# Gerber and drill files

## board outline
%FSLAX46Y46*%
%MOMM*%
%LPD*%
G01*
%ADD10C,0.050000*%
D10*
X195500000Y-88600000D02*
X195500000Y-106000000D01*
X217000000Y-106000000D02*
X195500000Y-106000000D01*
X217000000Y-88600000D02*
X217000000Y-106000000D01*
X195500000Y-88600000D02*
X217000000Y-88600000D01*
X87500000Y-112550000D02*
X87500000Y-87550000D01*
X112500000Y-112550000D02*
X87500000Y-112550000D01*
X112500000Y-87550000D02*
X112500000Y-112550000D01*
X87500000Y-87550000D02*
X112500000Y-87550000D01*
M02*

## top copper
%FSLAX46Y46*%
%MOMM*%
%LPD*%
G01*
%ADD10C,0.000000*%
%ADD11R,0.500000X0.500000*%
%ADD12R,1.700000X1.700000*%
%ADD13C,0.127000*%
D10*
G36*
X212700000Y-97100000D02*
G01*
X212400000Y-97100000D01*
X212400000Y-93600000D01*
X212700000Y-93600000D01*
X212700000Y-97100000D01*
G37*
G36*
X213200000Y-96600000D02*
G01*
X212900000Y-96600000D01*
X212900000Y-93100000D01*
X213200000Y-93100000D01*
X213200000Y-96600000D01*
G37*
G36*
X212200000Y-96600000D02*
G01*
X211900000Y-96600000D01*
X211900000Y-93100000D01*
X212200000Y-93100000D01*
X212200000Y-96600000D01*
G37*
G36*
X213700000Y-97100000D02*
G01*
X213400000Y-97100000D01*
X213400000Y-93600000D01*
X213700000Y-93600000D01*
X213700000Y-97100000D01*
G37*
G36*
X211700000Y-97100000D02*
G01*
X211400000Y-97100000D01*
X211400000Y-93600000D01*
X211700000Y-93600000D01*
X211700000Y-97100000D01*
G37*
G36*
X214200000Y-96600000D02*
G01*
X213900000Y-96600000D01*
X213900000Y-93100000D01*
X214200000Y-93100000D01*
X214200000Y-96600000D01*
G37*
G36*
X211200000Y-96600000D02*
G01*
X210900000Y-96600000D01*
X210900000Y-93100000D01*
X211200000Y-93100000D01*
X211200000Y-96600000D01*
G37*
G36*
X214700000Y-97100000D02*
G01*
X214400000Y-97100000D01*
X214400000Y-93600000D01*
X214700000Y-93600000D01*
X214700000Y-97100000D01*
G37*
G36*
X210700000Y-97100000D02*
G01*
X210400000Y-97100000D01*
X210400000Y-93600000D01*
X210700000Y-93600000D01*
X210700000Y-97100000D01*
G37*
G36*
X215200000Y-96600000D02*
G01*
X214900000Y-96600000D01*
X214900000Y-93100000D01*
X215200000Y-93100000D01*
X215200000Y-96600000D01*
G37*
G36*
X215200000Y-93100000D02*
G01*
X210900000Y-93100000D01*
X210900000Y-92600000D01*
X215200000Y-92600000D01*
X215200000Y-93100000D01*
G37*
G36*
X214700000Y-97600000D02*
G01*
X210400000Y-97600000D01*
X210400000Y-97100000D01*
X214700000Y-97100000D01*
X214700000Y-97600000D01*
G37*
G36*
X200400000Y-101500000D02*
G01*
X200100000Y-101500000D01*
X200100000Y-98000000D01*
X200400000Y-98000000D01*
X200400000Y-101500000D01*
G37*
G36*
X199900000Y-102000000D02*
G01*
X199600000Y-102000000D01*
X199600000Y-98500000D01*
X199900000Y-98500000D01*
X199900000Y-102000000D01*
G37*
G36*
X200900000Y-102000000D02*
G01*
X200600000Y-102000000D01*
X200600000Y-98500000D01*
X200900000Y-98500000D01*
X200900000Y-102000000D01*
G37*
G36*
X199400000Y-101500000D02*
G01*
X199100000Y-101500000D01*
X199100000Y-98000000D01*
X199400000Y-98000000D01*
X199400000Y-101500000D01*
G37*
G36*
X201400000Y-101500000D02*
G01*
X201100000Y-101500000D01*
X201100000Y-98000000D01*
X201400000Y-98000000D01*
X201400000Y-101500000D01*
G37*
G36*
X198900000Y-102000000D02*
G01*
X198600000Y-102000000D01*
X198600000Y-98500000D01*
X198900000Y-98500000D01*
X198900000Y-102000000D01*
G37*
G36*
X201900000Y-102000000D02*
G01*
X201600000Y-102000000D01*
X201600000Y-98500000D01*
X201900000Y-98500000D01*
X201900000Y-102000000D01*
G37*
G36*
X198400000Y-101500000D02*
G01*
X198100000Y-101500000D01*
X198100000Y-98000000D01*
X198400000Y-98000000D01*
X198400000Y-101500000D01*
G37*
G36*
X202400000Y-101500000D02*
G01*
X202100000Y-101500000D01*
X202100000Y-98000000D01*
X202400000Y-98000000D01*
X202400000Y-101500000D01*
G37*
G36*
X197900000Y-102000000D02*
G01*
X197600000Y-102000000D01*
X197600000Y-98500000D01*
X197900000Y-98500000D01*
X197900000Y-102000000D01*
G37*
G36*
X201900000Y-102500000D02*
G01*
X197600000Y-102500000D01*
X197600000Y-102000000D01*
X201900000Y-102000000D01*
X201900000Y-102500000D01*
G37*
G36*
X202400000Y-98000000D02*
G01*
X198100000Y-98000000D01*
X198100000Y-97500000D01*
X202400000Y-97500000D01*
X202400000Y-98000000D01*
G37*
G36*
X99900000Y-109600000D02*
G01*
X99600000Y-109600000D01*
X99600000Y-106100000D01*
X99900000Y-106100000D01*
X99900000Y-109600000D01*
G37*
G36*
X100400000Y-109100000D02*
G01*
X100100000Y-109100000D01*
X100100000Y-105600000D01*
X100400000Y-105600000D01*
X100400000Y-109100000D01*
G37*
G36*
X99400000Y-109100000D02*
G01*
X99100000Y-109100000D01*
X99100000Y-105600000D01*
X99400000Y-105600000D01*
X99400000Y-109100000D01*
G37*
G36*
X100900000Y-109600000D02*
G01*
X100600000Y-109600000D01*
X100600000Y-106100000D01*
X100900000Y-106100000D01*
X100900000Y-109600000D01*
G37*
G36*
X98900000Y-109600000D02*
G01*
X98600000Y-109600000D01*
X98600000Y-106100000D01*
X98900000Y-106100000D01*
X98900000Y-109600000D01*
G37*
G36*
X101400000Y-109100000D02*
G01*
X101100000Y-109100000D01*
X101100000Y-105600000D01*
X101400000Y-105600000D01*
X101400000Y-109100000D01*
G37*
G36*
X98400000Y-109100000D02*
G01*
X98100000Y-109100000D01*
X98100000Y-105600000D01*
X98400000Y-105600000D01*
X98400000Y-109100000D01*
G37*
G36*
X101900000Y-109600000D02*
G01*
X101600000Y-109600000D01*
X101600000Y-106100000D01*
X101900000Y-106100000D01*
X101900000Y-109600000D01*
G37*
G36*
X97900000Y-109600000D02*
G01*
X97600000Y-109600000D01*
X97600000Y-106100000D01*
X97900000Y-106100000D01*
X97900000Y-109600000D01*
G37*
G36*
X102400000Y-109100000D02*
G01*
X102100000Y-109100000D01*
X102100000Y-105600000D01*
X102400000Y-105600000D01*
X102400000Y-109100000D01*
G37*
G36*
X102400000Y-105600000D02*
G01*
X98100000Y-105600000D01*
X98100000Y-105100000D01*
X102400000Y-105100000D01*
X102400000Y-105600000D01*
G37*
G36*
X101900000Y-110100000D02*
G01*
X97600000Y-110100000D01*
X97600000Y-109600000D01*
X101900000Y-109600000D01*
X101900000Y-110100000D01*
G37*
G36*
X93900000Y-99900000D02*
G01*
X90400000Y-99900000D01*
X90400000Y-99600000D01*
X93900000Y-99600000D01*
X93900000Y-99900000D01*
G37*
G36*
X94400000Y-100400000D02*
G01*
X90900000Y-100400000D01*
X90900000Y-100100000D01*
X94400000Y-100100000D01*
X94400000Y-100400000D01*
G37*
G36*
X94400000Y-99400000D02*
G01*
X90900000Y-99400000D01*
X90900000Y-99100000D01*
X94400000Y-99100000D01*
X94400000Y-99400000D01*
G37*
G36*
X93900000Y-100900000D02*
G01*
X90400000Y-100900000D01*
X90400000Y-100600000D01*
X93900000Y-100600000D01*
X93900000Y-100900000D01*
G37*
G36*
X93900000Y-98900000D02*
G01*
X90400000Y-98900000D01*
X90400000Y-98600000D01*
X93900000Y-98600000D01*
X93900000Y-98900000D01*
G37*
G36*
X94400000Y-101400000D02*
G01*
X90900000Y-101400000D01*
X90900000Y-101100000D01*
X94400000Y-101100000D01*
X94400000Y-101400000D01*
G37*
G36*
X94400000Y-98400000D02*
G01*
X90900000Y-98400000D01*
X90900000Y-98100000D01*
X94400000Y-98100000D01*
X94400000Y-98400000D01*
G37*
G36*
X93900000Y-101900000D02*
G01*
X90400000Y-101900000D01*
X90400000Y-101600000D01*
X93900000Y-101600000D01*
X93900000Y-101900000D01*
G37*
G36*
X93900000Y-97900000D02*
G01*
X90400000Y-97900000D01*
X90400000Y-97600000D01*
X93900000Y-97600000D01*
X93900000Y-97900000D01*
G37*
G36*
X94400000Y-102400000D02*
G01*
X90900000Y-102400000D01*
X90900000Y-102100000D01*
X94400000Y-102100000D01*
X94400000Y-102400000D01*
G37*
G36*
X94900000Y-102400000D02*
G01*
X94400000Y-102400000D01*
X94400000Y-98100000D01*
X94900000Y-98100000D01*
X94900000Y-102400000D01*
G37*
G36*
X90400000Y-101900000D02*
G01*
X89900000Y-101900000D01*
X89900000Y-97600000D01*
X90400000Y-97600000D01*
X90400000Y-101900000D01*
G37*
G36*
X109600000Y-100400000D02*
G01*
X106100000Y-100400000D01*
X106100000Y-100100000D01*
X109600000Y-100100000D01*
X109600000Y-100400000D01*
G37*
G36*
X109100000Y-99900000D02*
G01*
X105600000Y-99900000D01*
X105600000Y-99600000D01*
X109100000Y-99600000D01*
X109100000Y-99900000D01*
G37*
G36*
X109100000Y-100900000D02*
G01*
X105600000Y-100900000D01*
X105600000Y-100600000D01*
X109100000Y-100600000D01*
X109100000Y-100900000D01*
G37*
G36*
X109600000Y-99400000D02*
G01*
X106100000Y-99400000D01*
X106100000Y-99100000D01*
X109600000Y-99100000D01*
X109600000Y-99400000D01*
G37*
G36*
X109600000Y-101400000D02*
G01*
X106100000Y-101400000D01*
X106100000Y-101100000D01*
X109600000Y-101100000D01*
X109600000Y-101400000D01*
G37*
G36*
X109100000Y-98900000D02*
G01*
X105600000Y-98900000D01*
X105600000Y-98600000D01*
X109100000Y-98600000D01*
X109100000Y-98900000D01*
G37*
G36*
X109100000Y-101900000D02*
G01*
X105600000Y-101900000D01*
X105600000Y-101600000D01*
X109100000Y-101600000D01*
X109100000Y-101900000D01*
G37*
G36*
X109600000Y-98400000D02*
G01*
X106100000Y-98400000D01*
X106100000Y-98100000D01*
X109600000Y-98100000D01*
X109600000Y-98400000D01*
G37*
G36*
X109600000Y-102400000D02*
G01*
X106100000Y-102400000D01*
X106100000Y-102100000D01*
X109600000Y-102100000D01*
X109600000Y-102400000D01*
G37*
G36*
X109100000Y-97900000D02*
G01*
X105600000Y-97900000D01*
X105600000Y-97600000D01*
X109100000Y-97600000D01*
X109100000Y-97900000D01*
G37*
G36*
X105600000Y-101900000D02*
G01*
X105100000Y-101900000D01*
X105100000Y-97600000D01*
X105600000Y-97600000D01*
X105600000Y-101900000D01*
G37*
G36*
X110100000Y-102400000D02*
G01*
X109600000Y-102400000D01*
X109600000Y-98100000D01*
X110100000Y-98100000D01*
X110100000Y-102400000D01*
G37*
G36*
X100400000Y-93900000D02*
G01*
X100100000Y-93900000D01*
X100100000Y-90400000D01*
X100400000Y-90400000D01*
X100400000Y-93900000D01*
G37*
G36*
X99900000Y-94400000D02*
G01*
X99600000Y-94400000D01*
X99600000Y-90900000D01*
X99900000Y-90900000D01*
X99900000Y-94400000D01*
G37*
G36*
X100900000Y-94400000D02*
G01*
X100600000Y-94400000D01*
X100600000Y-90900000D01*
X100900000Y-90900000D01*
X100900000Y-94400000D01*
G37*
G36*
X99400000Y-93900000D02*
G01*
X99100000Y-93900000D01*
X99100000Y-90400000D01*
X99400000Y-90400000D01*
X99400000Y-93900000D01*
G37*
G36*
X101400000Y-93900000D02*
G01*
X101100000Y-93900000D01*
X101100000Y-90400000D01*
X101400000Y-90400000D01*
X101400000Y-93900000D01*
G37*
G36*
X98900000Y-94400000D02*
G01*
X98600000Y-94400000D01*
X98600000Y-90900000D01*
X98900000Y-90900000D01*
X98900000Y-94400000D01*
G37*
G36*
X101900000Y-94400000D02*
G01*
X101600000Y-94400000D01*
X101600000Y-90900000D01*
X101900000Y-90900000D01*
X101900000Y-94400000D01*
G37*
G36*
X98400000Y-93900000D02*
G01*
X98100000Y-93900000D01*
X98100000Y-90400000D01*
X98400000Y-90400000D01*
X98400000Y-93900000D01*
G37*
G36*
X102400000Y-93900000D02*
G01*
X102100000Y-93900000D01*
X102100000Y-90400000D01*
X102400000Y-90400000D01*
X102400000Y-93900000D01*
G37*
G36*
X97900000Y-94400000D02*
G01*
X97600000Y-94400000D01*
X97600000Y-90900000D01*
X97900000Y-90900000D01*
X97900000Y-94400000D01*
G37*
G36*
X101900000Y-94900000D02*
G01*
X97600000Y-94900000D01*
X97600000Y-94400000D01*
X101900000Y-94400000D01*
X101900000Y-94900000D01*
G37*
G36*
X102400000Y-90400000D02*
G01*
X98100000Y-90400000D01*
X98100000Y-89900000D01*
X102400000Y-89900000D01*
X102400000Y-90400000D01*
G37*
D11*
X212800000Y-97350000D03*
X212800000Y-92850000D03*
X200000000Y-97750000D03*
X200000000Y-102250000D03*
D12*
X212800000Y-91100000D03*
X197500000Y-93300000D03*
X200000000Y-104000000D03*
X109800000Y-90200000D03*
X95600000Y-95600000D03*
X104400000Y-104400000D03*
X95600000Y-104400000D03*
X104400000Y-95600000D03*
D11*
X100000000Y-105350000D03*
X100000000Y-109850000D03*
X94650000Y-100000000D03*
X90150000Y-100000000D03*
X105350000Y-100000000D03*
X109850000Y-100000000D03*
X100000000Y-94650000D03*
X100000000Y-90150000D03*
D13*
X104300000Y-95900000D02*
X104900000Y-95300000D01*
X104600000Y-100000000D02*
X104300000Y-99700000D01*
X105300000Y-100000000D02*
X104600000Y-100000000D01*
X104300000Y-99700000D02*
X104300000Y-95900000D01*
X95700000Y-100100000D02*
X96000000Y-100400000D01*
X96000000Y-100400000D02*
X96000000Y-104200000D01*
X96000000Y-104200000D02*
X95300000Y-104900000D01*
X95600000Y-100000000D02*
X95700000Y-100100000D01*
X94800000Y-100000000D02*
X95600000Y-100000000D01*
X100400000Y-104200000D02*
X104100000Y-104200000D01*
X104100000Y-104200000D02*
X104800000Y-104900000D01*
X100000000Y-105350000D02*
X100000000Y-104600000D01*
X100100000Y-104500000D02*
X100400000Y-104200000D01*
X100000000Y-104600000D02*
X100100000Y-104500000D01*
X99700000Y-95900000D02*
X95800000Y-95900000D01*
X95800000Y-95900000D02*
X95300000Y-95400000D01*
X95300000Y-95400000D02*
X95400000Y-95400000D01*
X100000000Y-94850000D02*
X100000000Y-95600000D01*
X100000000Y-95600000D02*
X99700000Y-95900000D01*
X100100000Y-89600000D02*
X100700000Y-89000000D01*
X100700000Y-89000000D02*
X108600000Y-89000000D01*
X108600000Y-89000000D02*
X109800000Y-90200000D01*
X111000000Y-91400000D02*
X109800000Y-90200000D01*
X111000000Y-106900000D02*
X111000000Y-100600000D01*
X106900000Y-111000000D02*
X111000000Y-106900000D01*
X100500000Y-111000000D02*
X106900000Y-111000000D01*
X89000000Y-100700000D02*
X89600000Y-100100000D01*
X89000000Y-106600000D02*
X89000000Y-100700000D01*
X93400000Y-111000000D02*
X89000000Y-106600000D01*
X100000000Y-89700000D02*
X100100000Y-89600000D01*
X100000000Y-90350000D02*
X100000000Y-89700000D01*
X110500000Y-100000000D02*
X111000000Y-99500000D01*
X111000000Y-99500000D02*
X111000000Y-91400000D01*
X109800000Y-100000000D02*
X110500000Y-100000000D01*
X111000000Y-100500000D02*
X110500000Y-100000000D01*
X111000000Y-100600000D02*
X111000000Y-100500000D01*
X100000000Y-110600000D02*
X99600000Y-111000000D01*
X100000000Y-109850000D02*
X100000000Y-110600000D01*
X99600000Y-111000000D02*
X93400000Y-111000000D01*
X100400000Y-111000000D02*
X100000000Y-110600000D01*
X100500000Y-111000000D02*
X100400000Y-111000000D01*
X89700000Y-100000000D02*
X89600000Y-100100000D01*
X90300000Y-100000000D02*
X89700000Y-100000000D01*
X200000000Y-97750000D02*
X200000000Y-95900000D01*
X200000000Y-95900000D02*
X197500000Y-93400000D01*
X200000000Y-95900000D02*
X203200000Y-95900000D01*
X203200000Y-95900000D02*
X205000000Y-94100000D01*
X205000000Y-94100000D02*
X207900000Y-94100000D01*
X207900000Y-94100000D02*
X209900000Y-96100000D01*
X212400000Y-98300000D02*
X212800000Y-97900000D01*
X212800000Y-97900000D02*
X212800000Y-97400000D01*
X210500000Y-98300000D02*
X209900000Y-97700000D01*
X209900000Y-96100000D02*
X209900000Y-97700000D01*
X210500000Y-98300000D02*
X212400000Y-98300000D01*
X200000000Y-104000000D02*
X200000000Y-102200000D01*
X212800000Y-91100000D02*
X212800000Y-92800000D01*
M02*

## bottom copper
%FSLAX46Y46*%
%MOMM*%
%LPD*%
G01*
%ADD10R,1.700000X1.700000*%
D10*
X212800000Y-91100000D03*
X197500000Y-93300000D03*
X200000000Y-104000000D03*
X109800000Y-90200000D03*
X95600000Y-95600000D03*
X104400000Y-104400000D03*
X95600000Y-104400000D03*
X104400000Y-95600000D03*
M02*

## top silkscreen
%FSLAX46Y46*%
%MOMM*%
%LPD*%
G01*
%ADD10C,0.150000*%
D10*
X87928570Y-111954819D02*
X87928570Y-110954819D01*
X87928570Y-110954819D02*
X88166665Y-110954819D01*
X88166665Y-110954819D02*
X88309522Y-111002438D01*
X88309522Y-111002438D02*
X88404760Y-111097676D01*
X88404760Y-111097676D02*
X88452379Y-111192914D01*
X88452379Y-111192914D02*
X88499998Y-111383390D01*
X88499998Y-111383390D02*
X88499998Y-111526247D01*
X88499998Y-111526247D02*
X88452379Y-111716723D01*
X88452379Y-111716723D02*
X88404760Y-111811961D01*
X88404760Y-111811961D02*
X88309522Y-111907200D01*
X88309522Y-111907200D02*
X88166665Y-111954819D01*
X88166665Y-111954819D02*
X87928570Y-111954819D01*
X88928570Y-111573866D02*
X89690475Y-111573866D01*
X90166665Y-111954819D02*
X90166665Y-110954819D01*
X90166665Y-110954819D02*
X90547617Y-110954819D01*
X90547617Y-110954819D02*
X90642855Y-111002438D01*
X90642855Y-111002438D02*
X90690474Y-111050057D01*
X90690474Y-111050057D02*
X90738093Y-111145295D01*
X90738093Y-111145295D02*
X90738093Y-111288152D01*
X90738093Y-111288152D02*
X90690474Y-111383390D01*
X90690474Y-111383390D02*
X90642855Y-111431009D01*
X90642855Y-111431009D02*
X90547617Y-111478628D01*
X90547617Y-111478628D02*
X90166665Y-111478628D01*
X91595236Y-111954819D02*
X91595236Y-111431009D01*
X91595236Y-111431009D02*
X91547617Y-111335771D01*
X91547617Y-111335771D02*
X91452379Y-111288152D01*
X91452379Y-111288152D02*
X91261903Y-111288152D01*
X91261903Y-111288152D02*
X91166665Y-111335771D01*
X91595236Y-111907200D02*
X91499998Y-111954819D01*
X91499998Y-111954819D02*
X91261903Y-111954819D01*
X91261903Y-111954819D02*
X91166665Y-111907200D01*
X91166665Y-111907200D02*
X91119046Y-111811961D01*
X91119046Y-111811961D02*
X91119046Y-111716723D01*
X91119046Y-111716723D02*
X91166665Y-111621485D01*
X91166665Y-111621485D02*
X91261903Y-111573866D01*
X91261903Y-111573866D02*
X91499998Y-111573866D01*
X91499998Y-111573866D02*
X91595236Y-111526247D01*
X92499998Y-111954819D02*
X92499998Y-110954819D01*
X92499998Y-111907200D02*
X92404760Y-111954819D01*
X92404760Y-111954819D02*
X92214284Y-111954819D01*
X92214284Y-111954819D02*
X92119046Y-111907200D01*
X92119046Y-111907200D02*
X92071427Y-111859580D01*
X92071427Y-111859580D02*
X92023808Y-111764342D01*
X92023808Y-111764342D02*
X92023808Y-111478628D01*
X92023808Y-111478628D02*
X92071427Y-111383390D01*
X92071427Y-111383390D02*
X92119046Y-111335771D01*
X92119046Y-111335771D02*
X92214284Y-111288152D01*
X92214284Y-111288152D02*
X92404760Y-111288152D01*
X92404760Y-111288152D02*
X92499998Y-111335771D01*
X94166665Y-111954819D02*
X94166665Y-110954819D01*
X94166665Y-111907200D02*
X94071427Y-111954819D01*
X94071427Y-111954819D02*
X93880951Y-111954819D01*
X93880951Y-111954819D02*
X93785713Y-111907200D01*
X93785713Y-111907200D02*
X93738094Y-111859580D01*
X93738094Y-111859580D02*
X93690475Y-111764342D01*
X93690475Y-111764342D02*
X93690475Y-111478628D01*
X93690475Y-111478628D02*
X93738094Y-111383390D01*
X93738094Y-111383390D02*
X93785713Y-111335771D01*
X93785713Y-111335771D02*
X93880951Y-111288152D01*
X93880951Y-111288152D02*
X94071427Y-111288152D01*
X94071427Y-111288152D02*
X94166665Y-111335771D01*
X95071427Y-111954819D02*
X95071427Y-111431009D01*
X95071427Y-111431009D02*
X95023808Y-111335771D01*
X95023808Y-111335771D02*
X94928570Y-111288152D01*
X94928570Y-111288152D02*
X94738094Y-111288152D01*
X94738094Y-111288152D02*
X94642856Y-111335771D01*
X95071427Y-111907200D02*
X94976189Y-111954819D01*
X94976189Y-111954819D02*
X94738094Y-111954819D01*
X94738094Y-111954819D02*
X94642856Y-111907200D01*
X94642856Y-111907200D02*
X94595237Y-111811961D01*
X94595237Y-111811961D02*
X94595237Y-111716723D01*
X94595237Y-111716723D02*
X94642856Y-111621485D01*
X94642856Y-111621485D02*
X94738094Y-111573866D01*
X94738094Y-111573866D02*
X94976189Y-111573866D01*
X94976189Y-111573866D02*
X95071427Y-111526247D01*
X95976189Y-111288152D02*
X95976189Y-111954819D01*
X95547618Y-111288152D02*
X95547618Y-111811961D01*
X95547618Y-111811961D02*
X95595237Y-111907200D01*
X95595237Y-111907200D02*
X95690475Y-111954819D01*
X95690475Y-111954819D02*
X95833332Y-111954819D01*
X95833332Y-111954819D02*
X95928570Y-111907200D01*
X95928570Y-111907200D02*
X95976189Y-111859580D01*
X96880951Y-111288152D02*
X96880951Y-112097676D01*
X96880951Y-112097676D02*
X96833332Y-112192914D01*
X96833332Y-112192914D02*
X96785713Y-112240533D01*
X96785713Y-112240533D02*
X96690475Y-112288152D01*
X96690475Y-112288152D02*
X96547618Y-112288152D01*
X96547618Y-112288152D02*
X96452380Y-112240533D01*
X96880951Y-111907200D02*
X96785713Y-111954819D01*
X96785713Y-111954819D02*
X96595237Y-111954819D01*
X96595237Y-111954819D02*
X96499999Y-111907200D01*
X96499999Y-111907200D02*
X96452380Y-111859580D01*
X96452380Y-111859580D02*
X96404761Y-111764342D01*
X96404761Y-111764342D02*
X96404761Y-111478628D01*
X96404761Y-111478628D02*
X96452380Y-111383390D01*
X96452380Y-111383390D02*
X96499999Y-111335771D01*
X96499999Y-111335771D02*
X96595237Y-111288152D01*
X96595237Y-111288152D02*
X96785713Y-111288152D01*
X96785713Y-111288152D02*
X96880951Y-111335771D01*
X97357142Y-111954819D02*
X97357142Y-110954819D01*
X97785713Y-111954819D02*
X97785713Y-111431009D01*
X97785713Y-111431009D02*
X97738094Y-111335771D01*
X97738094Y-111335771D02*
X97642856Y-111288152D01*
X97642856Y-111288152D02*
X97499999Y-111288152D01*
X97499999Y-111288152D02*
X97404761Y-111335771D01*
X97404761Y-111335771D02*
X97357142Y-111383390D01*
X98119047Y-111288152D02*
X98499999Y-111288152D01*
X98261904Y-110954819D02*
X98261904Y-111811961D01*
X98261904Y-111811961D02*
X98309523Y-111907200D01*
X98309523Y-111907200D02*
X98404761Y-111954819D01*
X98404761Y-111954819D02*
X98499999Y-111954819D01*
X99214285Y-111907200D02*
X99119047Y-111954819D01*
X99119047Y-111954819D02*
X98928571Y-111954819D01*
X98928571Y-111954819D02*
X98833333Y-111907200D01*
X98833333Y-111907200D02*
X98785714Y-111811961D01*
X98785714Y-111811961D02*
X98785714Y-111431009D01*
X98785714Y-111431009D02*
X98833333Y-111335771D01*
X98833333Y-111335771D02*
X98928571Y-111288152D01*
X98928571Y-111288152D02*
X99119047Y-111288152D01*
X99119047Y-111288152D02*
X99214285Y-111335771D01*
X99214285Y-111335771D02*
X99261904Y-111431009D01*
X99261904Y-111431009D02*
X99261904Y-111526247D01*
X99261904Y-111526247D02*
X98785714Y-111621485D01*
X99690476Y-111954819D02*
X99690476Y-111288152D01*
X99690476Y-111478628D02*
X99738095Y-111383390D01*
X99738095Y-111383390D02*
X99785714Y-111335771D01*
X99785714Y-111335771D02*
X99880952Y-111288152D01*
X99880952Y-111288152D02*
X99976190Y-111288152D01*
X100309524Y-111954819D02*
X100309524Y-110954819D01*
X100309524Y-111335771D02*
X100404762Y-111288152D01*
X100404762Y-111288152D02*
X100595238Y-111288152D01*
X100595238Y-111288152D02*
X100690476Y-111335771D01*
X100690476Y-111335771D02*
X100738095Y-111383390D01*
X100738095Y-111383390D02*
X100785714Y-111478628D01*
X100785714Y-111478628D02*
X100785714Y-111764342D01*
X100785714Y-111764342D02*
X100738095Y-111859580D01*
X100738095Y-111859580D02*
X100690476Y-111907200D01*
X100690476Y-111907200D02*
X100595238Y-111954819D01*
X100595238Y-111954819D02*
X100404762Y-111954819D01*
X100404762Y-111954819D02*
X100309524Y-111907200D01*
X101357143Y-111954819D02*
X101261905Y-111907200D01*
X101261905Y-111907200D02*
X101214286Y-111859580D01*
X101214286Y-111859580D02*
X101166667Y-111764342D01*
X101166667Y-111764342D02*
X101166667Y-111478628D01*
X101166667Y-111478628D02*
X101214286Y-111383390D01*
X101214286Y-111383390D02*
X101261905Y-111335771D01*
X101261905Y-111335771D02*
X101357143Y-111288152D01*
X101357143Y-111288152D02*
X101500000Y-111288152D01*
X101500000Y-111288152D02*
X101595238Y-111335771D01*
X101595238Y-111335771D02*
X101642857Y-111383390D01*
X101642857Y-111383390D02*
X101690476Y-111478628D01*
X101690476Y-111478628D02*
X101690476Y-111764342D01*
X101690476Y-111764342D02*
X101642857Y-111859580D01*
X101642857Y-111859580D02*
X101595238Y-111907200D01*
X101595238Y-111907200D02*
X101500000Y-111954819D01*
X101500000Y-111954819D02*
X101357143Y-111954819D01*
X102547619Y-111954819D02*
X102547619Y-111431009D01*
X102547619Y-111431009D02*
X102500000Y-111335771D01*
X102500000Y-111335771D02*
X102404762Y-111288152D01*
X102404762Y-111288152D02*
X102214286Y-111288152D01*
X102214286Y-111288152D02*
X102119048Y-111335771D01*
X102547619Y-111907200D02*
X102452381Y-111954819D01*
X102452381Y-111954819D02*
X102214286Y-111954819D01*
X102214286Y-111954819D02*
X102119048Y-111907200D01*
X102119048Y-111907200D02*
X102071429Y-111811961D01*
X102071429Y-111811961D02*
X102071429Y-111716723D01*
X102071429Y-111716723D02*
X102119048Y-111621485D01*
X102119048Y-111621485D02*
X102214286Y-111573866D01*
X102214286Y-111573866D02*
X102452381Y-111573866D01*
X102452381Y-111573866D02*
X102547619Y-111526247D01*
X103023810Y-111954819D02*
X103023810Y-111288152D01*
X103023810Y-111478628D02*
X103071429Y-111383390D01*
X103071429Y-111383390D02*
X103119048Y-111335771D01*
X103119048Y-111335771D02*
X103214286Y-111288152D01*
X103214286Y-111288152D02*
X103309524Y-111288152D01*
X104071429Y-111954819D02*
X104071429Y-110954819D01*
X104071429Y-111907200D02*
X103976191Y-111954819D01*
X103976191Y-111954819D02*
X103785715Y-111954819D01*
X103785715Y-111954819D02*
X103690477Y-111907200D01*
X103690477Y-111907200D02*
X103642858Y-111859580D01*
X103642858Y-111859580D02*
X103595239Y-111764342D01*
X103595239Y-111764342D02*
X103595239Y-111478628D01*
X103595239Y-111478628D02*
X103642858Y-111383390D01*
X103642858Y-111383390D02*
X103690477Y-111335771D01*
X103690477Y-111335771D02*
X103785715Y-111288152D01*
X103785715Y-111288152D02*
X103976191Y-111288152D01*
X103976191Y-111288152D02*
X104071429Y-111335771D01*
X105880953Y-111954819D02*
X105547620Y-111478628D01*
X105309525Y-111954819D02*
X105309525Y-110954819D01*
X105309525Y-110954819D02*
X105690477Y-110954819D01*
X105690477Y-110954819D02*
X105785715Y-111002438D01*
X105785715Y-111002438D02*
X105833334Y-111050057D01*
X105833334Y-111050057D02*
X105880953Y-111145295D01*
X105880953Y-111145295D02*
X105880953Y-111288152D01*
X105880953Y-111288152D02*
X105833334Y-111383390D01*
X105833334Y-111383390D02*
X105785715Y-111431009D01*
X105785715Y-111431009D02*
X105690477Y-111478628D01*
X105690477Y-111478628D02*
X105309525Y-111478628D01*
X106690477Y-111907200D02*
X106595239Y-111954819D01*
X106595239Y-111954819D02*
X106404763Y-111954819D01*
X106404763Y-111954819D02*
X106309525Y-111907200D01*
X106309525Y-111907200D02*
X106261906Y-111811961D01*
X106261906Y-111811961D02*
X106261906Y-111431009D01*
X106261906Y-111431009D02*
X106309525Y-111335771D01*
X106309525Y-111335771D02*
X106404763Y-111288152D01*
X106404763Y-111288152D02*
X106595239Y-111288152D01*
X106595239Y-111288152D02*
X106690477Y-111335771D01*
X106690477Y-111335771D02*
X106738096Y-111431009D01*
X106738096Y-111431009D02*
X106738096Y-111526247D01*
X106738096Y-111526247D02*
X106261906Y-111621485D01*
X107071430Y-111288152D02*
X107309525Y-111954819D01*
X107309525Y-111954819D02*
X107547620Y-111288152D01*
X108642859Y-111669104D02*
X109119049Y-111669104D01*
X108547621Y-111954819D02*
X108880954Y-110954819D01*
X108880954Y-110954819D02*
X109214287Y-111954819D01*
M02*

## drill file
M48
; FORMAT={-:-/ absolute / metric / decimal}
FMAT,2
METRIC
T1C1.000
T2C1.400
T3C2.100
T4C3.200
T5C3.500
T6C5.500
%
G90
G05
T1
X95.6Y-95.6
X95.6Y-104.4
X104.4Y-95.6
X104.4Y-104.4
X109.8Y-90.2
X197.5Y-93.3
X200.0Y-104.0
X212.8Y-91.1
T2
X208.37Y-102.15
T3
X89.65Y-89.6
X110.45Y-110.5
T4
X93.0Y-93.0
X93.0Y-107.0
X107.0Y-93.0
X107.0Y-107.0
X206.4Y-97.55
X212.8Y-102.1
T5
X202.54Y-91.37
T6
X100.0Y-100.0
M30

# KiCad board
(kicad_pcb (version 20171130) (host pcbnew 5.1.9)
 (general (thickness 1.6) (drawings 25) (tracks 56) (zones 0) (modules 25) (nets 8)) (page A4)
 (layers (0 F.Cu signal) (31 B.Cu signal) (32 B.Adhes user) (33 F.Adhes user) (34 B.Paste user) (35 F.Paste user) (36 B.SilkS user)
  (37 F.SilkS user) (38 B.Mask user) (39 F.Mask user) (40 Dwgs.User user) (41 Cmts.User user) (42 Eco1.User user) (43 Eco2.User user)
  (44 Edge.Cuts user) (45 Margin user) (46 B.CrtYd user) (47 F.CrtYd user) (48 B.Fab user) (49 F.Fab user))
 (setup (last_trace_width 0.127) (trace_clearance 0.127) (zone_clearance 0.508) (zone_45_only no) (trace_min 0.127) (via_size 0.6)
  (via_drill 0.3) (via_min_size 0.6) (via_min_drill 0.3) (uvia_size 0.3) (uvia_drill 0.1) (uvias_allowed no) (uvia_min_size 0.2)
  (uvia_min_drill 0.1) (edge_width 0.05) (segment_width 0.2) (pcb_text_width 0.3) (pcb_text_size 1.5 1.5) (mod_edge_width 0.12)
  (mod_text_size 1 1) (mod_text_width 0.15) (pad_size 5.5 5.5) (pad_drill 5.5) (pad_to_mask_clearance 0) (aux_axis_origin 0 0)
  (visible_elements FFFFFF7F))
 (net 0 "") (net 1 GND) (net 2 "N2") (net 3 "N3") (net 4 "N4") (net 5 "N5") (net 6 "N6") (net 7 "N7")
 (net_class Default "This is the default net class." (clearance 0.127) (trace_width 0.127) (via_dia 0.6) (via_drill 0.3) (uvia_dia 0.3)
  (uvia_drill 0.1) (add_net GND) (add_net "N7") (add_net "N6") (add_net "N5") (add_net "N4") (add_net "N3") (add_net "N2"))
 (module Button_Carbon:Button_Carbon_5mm (layer F.Cu) (at 212.8 95.1)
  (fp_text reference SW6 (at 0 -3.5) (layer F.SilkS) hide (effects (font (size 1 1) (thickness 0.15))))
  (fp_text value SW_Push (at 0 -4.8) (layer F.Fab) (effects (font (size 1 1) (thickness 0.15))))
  (fp_poly (pts (xy -0.1 2) (xy -0.4 2) (xy -0.4 -1.5) (xy -0.1 -1.5)) (layer F.Cu) (width 0))
  (fp_poly (pts (xy 0.4 1.5) (xy 0.1 1.5) (xy 0.1 -2) (xy 0.4 -2)) (layer F.Cu) (width 0))
  (fp_poly (pts (xy -0.6 1.5) (xy -0.9 1.5) (xy -0.9 -2) (xy -0.6 -2)) (layer F.Cu) (width 0))
  (fp_poly (pts (xy 0.9 2) (xy 0.6 2) (xy 0.6 -1.5) (xy 0.9 -1.5)) (layer F.Cu) (width 0))
  (fp_poly (pts (xy -1.1 2) (xy -1.4 2) (xy -1.4 -1.5) (xy -1.1 -1.5)) (layer F.Cu) (width 0))
  (fp_poly (pts (xy 1.4 1.5) (xy 1.1 1.5) (xy 1.1 -2) (xy 1.4 -2)) (layer F.Cu) (width 0))
  (fp_poly (pts (xy -1.6 1.5) (xy -1.9 1.5) (xy -1.9 -2) (xy -1.6 -2)) (layer F.Cu) (width 0))
  (fp_poly (pts (xy 1.9 2) (xy 1.6 2) (xy 1.6 -1.5) (xy 1.9 -1.5)) (layer F.Cu) (width 0))
  (fp_poly (pts (xy -2.1 2) (xy -2.4 2) (xy -2.4 -1.5) (xy -2.1 -1.5)) (layer F.Cu) (width 0))
  (fp_poly (pts (xy 2.4 1.5) (xy 2.1 1.5) (xy 2.1 -2) (xy 2.4 -2)) (layer F.Cu) (width 0))
  (fp_poly (pts (xy 2.4 -2.5) (xy 2.4 -2) (xy -1.9 -2) (xy -1.9 -2.5)) (layer F.Cu) (width 0))
  (fp_poly (pts (xy 1.9 2) (xy 1.9 2.5) (xy -2.4 2.5) (xy -2.4 2)) (layer F.Cu) (width 0))
  (pad 2 smd rect (at 0 2.25) (size 0.5 0.5) (layers F.Cu F.Mask) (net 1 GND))
  (pad 1 smd rect (at 0 -2.25) (size 0.5 0.5) (layers F.Cu F.Mask) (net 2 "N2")))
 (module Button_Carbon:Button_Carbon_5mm (layer F.Cu) (at 200 100 180)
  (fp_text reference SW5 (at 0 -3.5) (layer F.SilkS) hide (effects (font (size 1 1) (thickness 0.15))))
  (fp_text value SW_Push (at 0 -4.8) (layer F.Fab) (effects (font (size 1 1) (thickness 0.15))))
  (fp_poly (pts (xy -0.1 2) (xy -0.4 2) (xy -0.4 -1.5) (xy -0.1 -1.5)) (layer F.Cu) (width 0))
  (fp_poly (pts (xy 0.4 1.5) (xy 0.1 1.5) (xy 0.1 -2) (xy 0.4 -2)) (layer F.Cu) (width 0))
  (fp_poly (pts (xy -0.6 1.5) (xy -0.9 1.5) (xy -0.9 -2) (xy -0.6 -2)) (layer F.Cu) (width 0))
  (fp_poly (pts (xy 0.9 2) (xy 0.6 2) (xy 0.6 -1.5) (xy 0.9 -1.5)) (layer F.Cu) (width 0))
  (fp_poly (pts (xy -1.1 2) (xy -1.4 2) (xy -1.4 -1.5) (xy -1.1 -1.5)) (layer F.Cu) (width 0))
  (fp_poly (pts (xy 1.4 1.5) (xy 1.1 1.5) (xy 1.1 -2) (xy 1.4 -2)) (layer F.Cu) (width 0))
  (fp_poly (pts (xy -1.6 1.5) (xy -1.9 1.5) (xy -1.9 -2) (xy -1.6 -2)) (layer F.Cu) (width 0))
  (fp_poly (pts (xy 1.9 2) (xy 1.6 2) (xy 1.6 -1.5) (xy 1.9 -1.5)) (layer F.Cu) (width 0))
  (fp_poly (pts (xy -2.1 2) (xy -2.4 2) (xy -2.4 -1.5) (xy -2.1 -1.5)) (layer F.Cu) (width 0))
  (fp_poly (pts (xy 2.4 1.5) (xy 2.1 1.5) (xy 2.1 -2) (xy 2.4 -2)) (layer F.Cu) (width 0))
  (fp_poly (pts (xy 2.4 -2.5) (xy 2.4 -2) (xy -1.9 -2) (xy -1.9 -2.5)) (layer F.Cu) (width 0))
  (fp_poly (pts (xy 1.9 2) (xy 1.9 2.5) (xy -2.4 2.5) (xy -2.4 2)) (layer F.Cu) (width 0))
  (pad 2 smd rect (at 0 2.25 180) (size 0.5 0.5) (layers F.Cu F.Mask) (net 1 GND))
  (pad 1 smd rect (at 0 -2.25 180) (size 0.5 0.5) (layers F.Cu F.Mask) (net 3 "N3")))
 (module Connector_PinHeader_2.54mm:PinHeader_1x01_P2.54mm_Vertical (layer B.Cu) (at 212.8 91.1)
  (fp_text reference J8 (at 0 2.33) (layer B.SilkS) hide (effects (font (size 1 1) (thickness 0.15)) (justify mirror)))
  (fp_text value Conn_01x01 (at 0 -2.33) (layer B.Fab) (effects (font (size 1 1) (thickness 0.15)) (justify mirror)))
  (pad 1 thru_hole rect (at 0 0) (size 1.7 1.7) (drill 1) (layers *.Cu *.Mask) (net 2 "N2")))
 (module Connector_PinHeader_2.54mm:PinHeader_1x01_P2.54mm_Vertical (layer B.Cu) (at 197.5 93.3)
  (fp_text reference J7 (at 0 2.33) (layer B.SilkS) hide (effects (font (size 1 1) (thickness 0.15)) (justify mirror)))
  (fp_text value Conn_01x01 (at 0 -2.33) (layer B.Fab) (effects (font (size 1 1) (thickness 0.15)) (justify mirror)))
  (pad 1 thru_hole rect (at 0 0) (size 1.7 1.7) (drill 1) (layers *.Cu *.Mask) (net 1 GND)))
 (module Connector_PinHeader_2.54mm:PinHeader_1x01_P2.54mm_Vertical (layer B.Cu) (at 200 104)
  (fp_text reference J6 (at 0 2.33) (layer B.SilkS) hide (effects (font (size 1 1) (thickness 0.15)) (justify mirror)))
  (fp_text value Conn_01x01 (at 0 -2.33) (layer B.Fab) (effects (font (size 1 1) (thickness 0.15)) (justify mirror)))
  (pad 1 thru_hole rect (at 0 0) (size 1.7 1.7) (drill 1) (layers *.Cu *.Mask) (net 3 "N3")))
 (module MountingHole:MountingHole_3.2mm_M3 (layer F.Cu) (at 212.8 102.1)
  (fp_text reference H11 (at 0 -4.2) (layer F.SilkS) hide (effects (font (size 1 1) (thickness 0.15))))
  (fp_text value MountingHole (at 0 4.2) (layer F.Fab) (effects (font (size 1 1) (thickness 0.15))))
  (pad 1 np_thru_hole circle (at 0 0) (size 3.2 3.2) (drill 3.2) (layers *.Cu *.Mask)))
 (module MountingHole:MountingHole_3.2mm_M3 (layer F.Cu) (at 206.4 97.55)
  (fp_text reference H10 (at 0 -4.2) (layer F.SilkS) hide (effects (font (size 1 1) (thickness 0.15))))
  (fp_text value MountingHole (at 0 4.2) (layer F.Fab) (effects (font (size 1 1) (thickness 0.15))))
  (pad 1 np_thru_hole circle (at 0 0) (size 3.2 3.2) (drill 3.2) (layers *.Cu *.Mask)))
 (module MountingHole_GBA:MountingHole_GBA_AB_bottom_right (layer F.Cu) (at 208.37 102.15)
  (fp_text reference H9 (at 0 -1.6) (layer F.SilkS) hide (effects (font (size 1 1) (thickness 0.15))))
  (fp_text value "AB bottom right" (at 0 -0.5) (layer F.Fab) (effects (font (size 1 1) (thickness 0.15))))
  (pad "" np_thru_hole circle (at 0 0 180) (size 1.4 1.4) (drill 1.4) (layers *.Cu *.Mask)))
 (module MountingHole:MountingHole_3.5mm (layer F.Cu) (at 202.54 91.37)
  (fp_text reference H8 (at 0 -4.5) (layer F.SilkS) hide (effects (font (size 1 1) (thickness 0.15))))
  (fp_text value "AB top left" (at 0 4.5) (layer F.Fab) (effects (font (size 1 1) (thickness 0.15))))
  (pad 1 np_thru_hole circle (at 0 0) (size 3.5 3.5) (drill 3.5) (layers *.Cu *.Mask)))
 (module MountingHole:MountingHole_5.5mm (layer F.Cu) (at 100 100)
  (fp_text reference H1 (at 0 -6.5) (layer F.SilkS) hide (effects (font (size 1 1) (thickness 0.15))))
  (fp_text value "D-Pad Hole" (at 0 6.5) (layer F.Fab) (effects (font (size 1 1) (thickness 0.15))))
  (pad 1 np_thru_hole circle (at 0 0) (size 5.5 5.5) (drill 5.5) (layers *.Cu *.Mask)))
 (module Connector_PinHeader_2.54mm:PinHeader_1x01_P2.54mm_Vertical (layer B.Cu) (at 109.8 90.2)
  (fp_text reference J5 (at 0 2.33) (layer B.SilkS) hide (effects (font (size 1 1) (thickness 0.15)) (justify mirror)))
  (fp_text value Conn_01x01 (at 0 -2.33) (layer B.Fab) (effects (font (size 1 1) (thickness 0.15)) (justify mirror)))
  (pad 1 thru_hole rect (at 0 0) (size 1.7 1.7) (drill 1) (layers *.Cu *.Mask) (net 1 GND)))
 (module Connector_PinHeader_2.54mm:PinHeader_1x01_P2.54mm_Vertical (layer B.Cu) (at 95.6 95.6)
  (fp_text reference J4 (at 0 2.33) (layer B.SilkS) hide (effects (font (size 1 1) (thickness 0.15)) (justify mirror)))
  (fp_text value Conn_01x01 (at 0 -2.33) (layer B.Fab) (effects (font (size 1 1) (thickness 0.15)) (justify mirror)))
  (pad 1 thru_hole rect (at 0 0) (size 1.7 1.7) (drill 1) (layers *.Cu *.Mask) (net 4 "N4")))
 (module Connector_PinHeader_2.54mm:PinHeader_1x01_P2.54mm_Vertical (layer B.Cu) (at 104.4 104.4)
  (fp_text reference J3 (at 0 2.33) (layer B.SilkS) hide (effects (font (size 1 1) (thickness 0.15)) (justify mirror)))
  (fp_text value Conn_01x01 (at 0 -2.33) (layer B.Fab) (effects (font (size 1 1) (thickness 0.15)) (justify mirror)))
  (pad 1 thru_hole rect (at 0 0) (size 1.7 1.7) (drill 1) (layers *.Cu *.Mask) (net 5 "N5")))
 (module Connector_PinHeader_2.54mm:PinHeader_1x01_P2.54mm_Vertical (layer B.Cu) (at 95.6 104.4)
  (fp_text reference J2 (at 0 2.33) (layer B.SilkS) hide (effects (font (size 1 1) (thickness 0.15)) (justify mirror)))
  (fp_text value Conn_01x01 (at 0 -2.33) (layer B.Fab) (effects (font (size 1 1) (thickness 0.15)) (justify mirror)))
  (pad 1 thru_hole rect (at 0 0) (size 1.7 1.7) (drill 1) (layers *.Cu *.Mask) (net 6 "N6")))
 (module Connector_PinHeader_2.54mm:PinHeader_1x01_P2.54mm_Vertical (layer B.Cu) (at 104.4 95.6)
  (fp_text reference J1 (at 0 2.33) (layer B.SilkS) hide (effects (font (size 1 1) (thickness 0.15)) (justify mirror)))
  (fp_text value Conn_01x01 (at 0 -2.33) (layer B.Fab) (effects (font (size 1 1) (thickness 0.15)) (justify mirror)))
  (pad 1 thru_hole rect (at 0 0) (size 1.7 1.7) (drill 1) (layers *.Cu *.Mask) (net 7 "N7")))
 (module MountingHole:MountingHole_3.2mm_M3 (layer F.Cu) (at 93 107)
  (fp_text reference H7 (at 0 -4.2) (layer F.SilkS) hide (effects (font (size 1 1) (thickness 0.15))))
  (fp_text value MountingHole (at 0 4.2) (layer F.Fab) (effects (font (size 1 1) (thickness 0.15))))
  (pad 1 np_thru_hole circle (at 0 0) (size 3.2 3.2) (drill 3.2) (layers *.Cu *.Mask)))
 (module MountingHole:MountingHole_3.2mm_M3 (layer F.Cu) (at 107 93)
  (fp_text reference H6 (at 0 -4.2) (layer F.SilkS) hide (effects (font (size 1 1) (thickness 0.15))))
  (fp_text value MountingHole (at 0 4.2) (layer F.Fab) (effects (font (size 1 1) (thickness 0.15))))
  (pad 1 np_thru_hole circle (at 0 0) (size 3.2 3.2) (drill 3.2) (layers *.Cu *.Mask)))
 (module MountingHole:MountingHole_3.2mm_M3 (layer F.Cu) (at 107 107)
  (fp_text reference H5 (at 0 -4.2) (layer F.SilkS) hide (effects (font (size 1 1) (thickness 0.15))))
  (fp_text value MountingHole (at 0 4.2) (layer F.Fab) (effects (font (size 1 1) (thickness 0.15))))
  (pad 1 np_thru_hole circle (at 0 0) (size 3.2 3.2) (drill 3.2) (layers *.Cu *.Mask)))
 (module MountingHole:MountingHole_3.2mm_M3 (layer F.Cu) (at 93 93)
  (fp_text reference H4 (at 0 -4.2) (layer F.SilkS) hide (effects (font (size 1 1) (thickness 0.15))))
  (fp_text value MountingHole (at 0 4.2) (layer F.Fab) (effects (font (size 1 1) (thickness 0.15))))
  (pad 1 np_thru_hole circle (at 0 0) (size 3.2 3.2) (drill 3.2) (layers *.Cu *.Mask)))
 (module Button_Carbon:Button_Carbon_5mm (layer F.Cu) (at 100 107.6)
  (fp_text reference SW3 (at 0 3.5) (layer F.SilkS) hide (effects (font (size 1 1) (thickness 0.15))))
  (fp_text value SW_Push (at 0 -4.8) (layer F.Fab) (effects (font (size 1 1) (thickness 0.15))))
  (fp_poly (pts (xy -0.1 2) (xy -0.4 2) (xy -0.4 -1.5) (xy -0.1 -1.5)) (layer F.Cu) (width 0))
  (fp_poly (pts (xy 0.4 1.5) (xy 0.1 1.5) (xy 0.1 -2) (xy 0.4 -2)) (layer F.Cu) (width 0))
  (fp_poly (pts (xy -0.6 1.5) (xy -0.9 1.5) (xy -0.9 -2) (xy -0.6 -2)) (layer F.Cu) (width 0))
  (fp_poly (pts (xy 0.9 2) (xy 0.6 2) (xy 0.6 -1.5) (xy 0.9 -1.5)) (layer F.Cu) (width 0))
  (fp_poly (pts (xy -1.1 2) (xy -1.4 2) (xy -1.4 -1.5) (xy -1.1 -1.5)) (layer F.Cu) (width 0))
  (fp_poly (pts (xy 1.4 1.5) (xy 1.1 1.5) (xy 1.1 -2) (xy 1.4 -2)) (layer F.Cu) (width 0))
  (fp_poly (pts (xy -1.6 1.5) (xy -1.9 1.5) (xy -1.9 -2) (xy -1.6 -2)) (layer F.Cu) (width 0))
  (fp_poly (pts (xy 1.9 2) (xy 1.6 2) (xy 1.6 -1.5) (xy 1.9 -1.5)) (layer F.Cu) (width 0))
  (fp_poly (pts (xy -2.1 2) (xy -2.4 2) (xy -2.4 -1.5) (xy -2.1 -1.5)) (layer F.Cu) (width 0))
  (fp_poly (pts (xy 2.4 1.5) (xy 2.1 1.5) (xy 2.1 -2) (xy 2.4 -2)) (layer F.Cu) (width 0))
  (fp_poly (pts (xy 2.4 -2.5) (xy 2.4 -2) (xy -1.9 -2) (xy -1.9 -2.5)) (layer F.Cu) (width 0))
  (fp_poly (pts (xy 1.9 2) (xy 1.9 2.5) (xy -2.4 2.5) (xy -2.4 2)) (layer F.Cu) (width 0))
  (pad 1 smd rect (at 0 -2.25) (size 0.5 0.5) (layers F.Cu F.Mask) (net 5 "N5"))
  (pad 2 smd rect (at 0 2.25) (size 0.5 0.5) (layers F.Cu F.Mask) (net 1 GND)))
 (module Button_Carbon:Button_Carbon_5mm (layer F.Cu) (at 92.4 100 270)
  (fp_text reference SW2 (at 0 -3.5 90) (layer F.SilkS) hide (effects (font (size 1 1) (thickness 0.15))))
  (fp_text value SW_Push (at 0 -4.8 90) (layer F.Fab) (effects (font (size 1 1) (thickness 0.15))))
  (fp_poly (pts (xy -0.1 2) (xy -0.4 2) (xy -0.4 -1.5) (xy -0.1 -1.5)) (layer F.Cu) (width 0))
  (fp_poly (pts (xy 0.4 1.5) (xy 0.1 1.5) (xy 0.1 -2) (xy 0.4 -2)) (layer F.Cu) (width 0))
  (fp_poly (pts (xy -0.6 1.5) (xy -0.9 1.5) (xy -0.9 -2) (xy -0.6 -2)) (layer F.Cu) (width 0))
  (fp_poly (pts (xy 0.9 2) (xy 0.6 2) (xy 0.6 -1.5) (xy 0.9 -1.5)) (layer F.Cu) (width 0))
  (fp_poly (pts (xy -1.1 2) (xy -1.4 2) (xy -1.4 -1.5) (xy -1.1 -1.5)) (layer F.Cu) (width 0))
  (fp_poly (pts (xy 1.4 1.5) (xy 1.1 1.5) (xy 1.1 -2) (xy 1.4 -2)) (layer F.Cu) (width 0))
  (fp_poly (pts (xy -1.6 1.5) (xy -1.9 1.5) (xy -1.9 -2) (xy -1.6 -2)) (layer F.Cu) (width 0))
  (fp_poly (pts (xy 1.9 2) (xy 1.6 2) (xy 1.6 -1.5) (xy 1.9 -1.5)) (layer F.Cu) (width 0))
  (fp_poly (pts (xy -2.1 2) (xy -2.4 2) (xy -2.4 -1.5) (xy -2.1 -1.5)) (layer F.Cu) (width 0))
  (fp_poly (pts (xy 2.4 1.5) (xy 2.1 1.5) (xy 2.1 -2) (xy 2.4 -2)) (layer F.Cu) (width 0))
  (fp_poly (pts (xy 2.4 -2.5) (xy 2.4 -2) (xy -1.9 -2) (xy -1.9 -2.5)) (layer F.Cu) (width 0))
  (fp_poly (pts (xy 1.9 2) (xy 1.9 2.5) (xy -2.4 2.5) (xy -2.4 2)) (layer F.Cu) (width 0))
  (pad 1 smd rect (at 0 -2.25 270) (size 0.5 0.5) (layers F.Cu F.Mask) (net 6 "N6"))
  (pad 2 smd rect (at 0 2.25 270) (size 0.5 0.5) (layers F.Cu F.Mask) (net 1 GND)))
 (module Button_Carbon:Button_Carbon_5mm (layer F.Cu) (at 107.6 100 90)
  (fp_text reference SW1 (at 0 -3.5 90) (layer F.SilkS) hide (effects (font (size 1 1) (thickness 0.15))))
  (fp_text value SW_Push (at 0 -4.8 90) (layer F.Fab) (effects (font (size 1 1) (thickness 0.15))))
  (fp_poly (pts (xy -0.1 2) (xy -0.4 2) (xy -0.4 -1.5) (xy -0.1 -1.5)) (layer F.Cu) (width 0))
  (fp_poly (pts (xy 0.4 1.5) (xy 0.1 1.5) (xy 0.1 -2) (xy 0.4 -2)) (layer F.Cu) (width 0))
  (fp_poly (pts (xy -0.6 1.5) (xy -0.9 1.5) (xy -0.9 -2) (xy -0.6 -2)) (layer F.Cu) (width 0))
  (fp_poly (pts (xy 0.9 2) (xy 0.6 2) (xy 0.6 -1.5) (xy 0.9 -1.5)) (layer F.Cu) (width 0))
  (fp_poly (pts (xy -1.1 2) (xy -1.4 2) (xy -1.4 -1.5) (xy -1.1 -1.5)) (layer F.Cu) (width 0))
  (fp_poly (pts (xy 1.4 1.5) (xy 1.1 1.5) (xy 1.1 -2) (xy 1.4 -2)) (layer F.Cu) (width 0))
  (fp_poly (pts (xy -1.6 1.5) (xy -1.9 1.5) (xy -1.9 -2) (xy -1.6 -2)) (layer F.Cu) (width 0))
  (fp_poly (pts (xy 1.9 2) (xy 1.6 2) (xy 1.6 -1.5) (xy 1.9 -1.5)) (layer F.Cu) (width 0))
  (fp_poly (pts (xy -2.1 2) (xy -2.4 2) (xy -2.4 -1.5) (xy -2.1 -1.5)) (layer F.Cu) (width 0))
  (fp_poly (pts (xy 2.4 1.5) (xy 2.1 1.5) (xy 2.1 -2) (xy 2.4 -2)) (layer F.Cu) (width 0))
  (fp_poly (pts (xy 2.4 -2.5) (xy 2.4 -2) (xy -1.9 -2) (xy -1.9 -2.5)) (layer F.Cu) (width 0))
  (fp_poly (pts (xy 1.9 2) (xy 1.9 2.5) (xy -2.4 2.5) (xy -2.4 2)) (layer F.Cu) (width 0))
  (pad 1 smd rect (at 0 -2.25 90) (size 0.5 0.5) (layers F.Cu F.Mask) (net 7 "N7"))
  (pad 2 smd rect (at 0 2.25 90) (size 0.5 0.5) (layers F.Cu F.Mask) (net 1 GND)))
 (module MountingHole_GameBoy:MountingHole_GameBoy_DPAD (layer F.Cu) (at 110.45 110.5)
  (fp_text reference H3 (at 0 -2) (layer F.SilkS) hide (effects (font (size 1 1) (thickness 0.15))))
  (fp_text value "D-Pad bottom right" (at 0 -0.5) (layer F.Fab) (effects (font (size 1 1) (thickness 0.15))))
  (pad "" np_thru_hole circle (at 0 0 180) (size 2.1 2.1) (drill 2.1) (layers *.Cu *.Mask)))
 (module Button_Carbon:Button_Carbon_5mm (layer F.Cu) (at 100 92.4 180) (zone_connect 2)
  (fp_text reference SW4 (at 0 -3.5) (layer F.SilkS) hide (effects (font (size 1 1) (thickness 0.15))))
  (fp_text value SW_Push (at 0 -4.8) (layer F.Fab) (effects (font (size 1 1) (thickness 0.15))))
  (fp_poly (pts (xy -0.1 2) (xy -0.4 2) (xy -0.4 -1.5) (xy -0.1 -1.5)) (layer F.Cu) (width 0))
  (fp_poly (pts (xy 0.4 1.5) (xy 0.1 1.5) (xy 0.1 -2) (xy 0.4 -2)) (layer F.Cu) (width 0))
  (fp_poly (pts (xy -0.6 1.5) (xy -0.9 1.5) (xy -0.9 -2) (xy -0.6 -2)) (layer F.Cu) (width 0))
  (fp_poly (pts (xy 0.9 2) (xy 0.6 2) (xy 0.6 -1.5) (xy 0.9 -1.5)) (layer F.Cu) (width 0))
  (fp_poly (pts (xy -1.1 2) (xy -1.4 2) (xy -1.4 -1.5) (xy -1.1 -1.5)) (layer F.Cu) (width 0))
  (fp_poly (pts (xy 1.4 1.5) (xy 1.1 1.5) (xy 1.1 -2) (xy 1.4 -2)) (layer F.Cu) (width 0))
  (fp_poly (pts (xy -1.6 1.5) (xy -1.9 1.5) (xy -1.9 -2) (xy -1.6 -2)) (layer F.Cu) (width 0))
  (fp_poly (pts (xy 1.9 2) (xy 1.6 2) (xy 1.6 -1.5) (xy 1.9 -1.5)) (layer F.Cu) (width 0))
  (fp_poly (pts (xy -2.1 2) (xy -2.4 2) (xy -2.4 -1.5) (xy -2.1 -1.5)) (layer F.Cu) (width 0))
  (fp_poly (pts (xy 2.4 1.5) (xy 2.1 1.5) (xy 2.1 -2) (xy 2.4 -2)) (layer F.Cu) (width 0))
  (fp_poly (pts (xy 2.4 -2.5) (xy 2.4 -2) (xy -1.9 -2) (xy -1.9 -2.5)) (layer F.Cu) (width 0))
  (fp_poly (pts (xy 1.9 2) (xy 1.9 2.5) (xy -2.4 2.5) (xy -2.4 2)) (layer F.Cu) (width 0))
  (pad 1 smd rect (at 0 -2.25 180) (size 0.5 0.5) (layers F.Cu F.Mask) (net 4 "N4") (zone_connect 2))
  (pad 2 smd rect (at 0 2.25 180) (size 0.5 0.5) (layers F.Cu F.Mask) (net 1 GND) (zone_connect 2)))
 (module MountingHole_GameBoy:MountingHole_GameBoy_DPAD (layer F.Cu) (at 89.65 89.6 180)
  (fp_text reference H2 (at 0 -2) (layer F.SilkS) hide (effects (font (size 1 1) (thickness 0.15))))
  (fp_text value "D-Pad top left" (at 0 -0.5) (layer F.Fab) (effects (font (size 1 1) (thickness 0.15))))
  (pad "" np_thru_hole circle (at 0 0) (size 2.1 2.1) (drill 2.1) (layers *.Cu *.Mask)))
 (gr_line (start 195.5 88.6) (end 195.5 106) (layer Edge.Cuts) (width 0.05))
 (gr_line (start 217 106) (end 195.5 106) (layer Edge.Cuts) (width 0.05))
 (gr_line (start 217 88.6) (end 217 106) (layer Edge.Cuts) (width 0.05))
 (gr_line (start 195.5 88.6) (end 217 88.6) (layer Edge.Cuts) (width 0.05))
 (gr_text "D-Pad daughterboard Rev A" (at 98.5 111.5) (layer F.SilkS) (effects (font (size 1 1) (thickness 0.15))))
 (gr_line (start 87.5 112.55) (end 87.5 87.55) (layer Edge.Cuts) (width 0.05))
 (gr_line (start 112.5 112.55) (end 87.5 112.55) (layer Edge.Cuts) (width 0.05))
 (gr_line (start 112.5 87.55) (end 112.5 112.55) (layer Edge.Cuts) (width 0.05))
 (gr_line (start 87.5 87.55) (end 112.5 87.55) (layer Edge.Cuts) (width 0.05))
 (segment (start 104.3 95.9) (end 104.9 95.3) (width 0.127) (layer F.Cu) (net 7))
 (segment (start 104.6 100) (end 104.3 99.7) (width 0.127) (layer F.Cu) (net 7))
 (segment (start 105.3 100) (end 104.6 100) (width 0.127) (layer F.Cu) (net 7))
 (segment (start 104.3 99.7) (end 104.3 95.9) (width 0.127) (layer F.Cu) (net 7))
 (segment (start 95.7 100.1) (end 96 100.4) (width 0.127) (layer F.Cu) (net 6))
 (segment (start 96 100.4) (end 96 104.2) (width 0.127) (layer F.Cu) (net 6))
 (segment (start 96 104.2) (end 95.3 104.9) (width 0.127) (layer F.Cu) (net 6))
 (segment (start 95.6 100) (end 95.7 100.1) (width 0.127) (layer F.Cu) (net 6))
 (segment (start 94.8 100) (end 95.6 100) (width 0.127) (layer F.Cu) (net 6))
 (segment (start 100.4 104.2) (end 104.1 104.2) (width 0.127) (layer F.Cu) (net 5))
 (segment (start 104.1 104.2) (end 104.8 104.9) (width 0.127) (layer F.Cu) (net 5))
 (segment (start 100 105.35) (end 100 104.6) (width 0.127) (layer F.Cu) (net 5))
 (segment (start 100.1 104.5) (end 100.4 104.2) (width 0.127) (layer F.Cu) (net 5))
 (segment (start 100 104.6) (end 100.1 104.5) (width 0.127) (layer F.Cu) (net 5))
 (segment (start 99.7 95.9) (end 95.8 95.9) (width 0.127) (layer F.Cu) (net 4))
 (segment (start 95.8 95.9) (end 95.3 95.4) (width 0.127) (layer F.Cu) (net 4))
 (segment (start 95.3 95.4) (end 95.4 95.4) (width 0.127) (layer F.Cu) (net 4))
 (segment (start 100 94.85) (end 100 95.6) (width 0.127) (layer F.Cu) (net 4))
 (segment (start 100 95.6) (end 99.7 95.9) (width 0.127) (layer F.Cu) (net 4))
 (segment (start 100.1 89.6) (end 100.7 89) (width 0.127) (layer F.Cu) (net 1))
 (segment (start 100.7 89) (end 108.6 89) (width 0.127) (layer F.Cu) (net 1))
 (segment (start 108.6 89) (end 109.8 90.2) (width 0.127) (layer F.Cu) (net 1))
 (segment (start 111 91.4) (end 109.8 90.2) (width 0.127) (layer F.Cu) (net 1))
 (segment (start 111 106.9) (end 111 100.6) (width 0.127) (layer F.Cu) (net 1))
 (segment (start 106.9 111) (end 111 106.9) (width 0.127) (layer F.Cu) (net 1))
 (segment (start 100.5 111) (end 106.9 111) (width 0.127) (layer F.Cu) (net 1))
 (segment (start 89 100.7) (end 89.6 100.1) (width 0.127) (layer F.Cu) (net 1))
 (segment (start 89 106.6) (end 89 100.7) (width 0.127) (layer F.Cu) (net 1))
 (segment (start 93.4 111) (end 89 106.6) (width 0.127) (layer F.Cu) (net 1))
 (segment (start 100 89.7) (end 100.1 89.6) (width 0.127) (layer F.Cu) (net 1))
 (segment (start 100 90.35) (end 100 89.7) (width 0.127) (layer F.Cu) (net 1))
 (segment (start 110.5 100) (end 111 99.5) (width 0.127) (layer F.Cu) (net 1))
 (segment (start 111 99.5) (end 111 91.4) (width 0.127) (layer F.Cu) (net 1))
 (segment (start 109.8 100) (end 110.5 100) (width 0.127) (layer F.Cu) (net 1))
 (segment (start 111 100.5) (end 110.5 100) (width 0.127) (layer F.Cu) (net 1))
 (segment (start 111 100.6) (end 111 100.5) (width 0.127) (layer F.Cu) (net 1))
 (segment (start 100 110.6) (end 99.6 111) (width 0.127) (layer F.Cu) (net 1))
 (segment (start 100 109.85) (end 100 110.6) (width 0.127) (layer F.Cu) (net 1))
 (segment (start 99.6 111) (end 93.4 111) (width 0.127) (layer F.Cu) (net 1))
 (segment (start 100.4 111) (end 100 110.6) (width 0.127) (layer F.Cu) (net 1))
 (segment (start 100.5 111) (end 100.4 111) (width 0.127) (layer F.Cu) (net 1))
 (segment (start 89.7 100) (end 89.6 100.1) (width 0.127) (layer F.Cu) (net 1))
 (segment (start 90.3 100) (end 89.7 100) (width 0.127) (layer F.Cu) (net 1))
 (segment (start 200 97.75) (end 200 95.9) (width 0.127) (layer F.Cu) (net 1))
 (segment (start 200 95.9) (end 197.5 93.4) (width 0.127) (layer F.Cu) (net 1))
 (segment (start 200 95.9) (end 203.2 95.9) (width 0.127) (layer F.Cu) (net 1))
 (segment (start 203.2 95.9) (end 205 94.1) (width 0.127) (layer F.Cu) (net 1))
 (segment (start 205 94.1) (end 207.9 94.1) (width 0.127) (layer F.Cu) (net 1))
 (segment (start 207.9 94.1) (end 209.9 96.1) (width 0.127) (layer F.Cu) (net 1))
 (segment (start 212.4 98.3) (end 212.8 97.9) (width 0.127) (layer F.Cu) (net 1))
 (segment (start 212.8 97.9) (end 212.8 97.4) (width 0.127) (layer F.Cu) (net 1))
 (segment (start 210.5 98.3) (end 209.9 97.7) (width 0.127) (layer F.Cu) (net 1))
 (segment (start 209.9 96.1) (end 209.9 97.7) (width 0.127) (layer F.Cu) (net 1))
 (segment (start 210.5 98.3) (end 212.4 98.3) (width 0.127) (layer F.Cu) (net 1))
 (segment (start 200 104) (end 200 102.2) (width 0.127) (layer F.Cu) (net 3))
 (segment (start 212.8 91.1) (end 212.8 92.8) (width 0.127) (layer F.Cu) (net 2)))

